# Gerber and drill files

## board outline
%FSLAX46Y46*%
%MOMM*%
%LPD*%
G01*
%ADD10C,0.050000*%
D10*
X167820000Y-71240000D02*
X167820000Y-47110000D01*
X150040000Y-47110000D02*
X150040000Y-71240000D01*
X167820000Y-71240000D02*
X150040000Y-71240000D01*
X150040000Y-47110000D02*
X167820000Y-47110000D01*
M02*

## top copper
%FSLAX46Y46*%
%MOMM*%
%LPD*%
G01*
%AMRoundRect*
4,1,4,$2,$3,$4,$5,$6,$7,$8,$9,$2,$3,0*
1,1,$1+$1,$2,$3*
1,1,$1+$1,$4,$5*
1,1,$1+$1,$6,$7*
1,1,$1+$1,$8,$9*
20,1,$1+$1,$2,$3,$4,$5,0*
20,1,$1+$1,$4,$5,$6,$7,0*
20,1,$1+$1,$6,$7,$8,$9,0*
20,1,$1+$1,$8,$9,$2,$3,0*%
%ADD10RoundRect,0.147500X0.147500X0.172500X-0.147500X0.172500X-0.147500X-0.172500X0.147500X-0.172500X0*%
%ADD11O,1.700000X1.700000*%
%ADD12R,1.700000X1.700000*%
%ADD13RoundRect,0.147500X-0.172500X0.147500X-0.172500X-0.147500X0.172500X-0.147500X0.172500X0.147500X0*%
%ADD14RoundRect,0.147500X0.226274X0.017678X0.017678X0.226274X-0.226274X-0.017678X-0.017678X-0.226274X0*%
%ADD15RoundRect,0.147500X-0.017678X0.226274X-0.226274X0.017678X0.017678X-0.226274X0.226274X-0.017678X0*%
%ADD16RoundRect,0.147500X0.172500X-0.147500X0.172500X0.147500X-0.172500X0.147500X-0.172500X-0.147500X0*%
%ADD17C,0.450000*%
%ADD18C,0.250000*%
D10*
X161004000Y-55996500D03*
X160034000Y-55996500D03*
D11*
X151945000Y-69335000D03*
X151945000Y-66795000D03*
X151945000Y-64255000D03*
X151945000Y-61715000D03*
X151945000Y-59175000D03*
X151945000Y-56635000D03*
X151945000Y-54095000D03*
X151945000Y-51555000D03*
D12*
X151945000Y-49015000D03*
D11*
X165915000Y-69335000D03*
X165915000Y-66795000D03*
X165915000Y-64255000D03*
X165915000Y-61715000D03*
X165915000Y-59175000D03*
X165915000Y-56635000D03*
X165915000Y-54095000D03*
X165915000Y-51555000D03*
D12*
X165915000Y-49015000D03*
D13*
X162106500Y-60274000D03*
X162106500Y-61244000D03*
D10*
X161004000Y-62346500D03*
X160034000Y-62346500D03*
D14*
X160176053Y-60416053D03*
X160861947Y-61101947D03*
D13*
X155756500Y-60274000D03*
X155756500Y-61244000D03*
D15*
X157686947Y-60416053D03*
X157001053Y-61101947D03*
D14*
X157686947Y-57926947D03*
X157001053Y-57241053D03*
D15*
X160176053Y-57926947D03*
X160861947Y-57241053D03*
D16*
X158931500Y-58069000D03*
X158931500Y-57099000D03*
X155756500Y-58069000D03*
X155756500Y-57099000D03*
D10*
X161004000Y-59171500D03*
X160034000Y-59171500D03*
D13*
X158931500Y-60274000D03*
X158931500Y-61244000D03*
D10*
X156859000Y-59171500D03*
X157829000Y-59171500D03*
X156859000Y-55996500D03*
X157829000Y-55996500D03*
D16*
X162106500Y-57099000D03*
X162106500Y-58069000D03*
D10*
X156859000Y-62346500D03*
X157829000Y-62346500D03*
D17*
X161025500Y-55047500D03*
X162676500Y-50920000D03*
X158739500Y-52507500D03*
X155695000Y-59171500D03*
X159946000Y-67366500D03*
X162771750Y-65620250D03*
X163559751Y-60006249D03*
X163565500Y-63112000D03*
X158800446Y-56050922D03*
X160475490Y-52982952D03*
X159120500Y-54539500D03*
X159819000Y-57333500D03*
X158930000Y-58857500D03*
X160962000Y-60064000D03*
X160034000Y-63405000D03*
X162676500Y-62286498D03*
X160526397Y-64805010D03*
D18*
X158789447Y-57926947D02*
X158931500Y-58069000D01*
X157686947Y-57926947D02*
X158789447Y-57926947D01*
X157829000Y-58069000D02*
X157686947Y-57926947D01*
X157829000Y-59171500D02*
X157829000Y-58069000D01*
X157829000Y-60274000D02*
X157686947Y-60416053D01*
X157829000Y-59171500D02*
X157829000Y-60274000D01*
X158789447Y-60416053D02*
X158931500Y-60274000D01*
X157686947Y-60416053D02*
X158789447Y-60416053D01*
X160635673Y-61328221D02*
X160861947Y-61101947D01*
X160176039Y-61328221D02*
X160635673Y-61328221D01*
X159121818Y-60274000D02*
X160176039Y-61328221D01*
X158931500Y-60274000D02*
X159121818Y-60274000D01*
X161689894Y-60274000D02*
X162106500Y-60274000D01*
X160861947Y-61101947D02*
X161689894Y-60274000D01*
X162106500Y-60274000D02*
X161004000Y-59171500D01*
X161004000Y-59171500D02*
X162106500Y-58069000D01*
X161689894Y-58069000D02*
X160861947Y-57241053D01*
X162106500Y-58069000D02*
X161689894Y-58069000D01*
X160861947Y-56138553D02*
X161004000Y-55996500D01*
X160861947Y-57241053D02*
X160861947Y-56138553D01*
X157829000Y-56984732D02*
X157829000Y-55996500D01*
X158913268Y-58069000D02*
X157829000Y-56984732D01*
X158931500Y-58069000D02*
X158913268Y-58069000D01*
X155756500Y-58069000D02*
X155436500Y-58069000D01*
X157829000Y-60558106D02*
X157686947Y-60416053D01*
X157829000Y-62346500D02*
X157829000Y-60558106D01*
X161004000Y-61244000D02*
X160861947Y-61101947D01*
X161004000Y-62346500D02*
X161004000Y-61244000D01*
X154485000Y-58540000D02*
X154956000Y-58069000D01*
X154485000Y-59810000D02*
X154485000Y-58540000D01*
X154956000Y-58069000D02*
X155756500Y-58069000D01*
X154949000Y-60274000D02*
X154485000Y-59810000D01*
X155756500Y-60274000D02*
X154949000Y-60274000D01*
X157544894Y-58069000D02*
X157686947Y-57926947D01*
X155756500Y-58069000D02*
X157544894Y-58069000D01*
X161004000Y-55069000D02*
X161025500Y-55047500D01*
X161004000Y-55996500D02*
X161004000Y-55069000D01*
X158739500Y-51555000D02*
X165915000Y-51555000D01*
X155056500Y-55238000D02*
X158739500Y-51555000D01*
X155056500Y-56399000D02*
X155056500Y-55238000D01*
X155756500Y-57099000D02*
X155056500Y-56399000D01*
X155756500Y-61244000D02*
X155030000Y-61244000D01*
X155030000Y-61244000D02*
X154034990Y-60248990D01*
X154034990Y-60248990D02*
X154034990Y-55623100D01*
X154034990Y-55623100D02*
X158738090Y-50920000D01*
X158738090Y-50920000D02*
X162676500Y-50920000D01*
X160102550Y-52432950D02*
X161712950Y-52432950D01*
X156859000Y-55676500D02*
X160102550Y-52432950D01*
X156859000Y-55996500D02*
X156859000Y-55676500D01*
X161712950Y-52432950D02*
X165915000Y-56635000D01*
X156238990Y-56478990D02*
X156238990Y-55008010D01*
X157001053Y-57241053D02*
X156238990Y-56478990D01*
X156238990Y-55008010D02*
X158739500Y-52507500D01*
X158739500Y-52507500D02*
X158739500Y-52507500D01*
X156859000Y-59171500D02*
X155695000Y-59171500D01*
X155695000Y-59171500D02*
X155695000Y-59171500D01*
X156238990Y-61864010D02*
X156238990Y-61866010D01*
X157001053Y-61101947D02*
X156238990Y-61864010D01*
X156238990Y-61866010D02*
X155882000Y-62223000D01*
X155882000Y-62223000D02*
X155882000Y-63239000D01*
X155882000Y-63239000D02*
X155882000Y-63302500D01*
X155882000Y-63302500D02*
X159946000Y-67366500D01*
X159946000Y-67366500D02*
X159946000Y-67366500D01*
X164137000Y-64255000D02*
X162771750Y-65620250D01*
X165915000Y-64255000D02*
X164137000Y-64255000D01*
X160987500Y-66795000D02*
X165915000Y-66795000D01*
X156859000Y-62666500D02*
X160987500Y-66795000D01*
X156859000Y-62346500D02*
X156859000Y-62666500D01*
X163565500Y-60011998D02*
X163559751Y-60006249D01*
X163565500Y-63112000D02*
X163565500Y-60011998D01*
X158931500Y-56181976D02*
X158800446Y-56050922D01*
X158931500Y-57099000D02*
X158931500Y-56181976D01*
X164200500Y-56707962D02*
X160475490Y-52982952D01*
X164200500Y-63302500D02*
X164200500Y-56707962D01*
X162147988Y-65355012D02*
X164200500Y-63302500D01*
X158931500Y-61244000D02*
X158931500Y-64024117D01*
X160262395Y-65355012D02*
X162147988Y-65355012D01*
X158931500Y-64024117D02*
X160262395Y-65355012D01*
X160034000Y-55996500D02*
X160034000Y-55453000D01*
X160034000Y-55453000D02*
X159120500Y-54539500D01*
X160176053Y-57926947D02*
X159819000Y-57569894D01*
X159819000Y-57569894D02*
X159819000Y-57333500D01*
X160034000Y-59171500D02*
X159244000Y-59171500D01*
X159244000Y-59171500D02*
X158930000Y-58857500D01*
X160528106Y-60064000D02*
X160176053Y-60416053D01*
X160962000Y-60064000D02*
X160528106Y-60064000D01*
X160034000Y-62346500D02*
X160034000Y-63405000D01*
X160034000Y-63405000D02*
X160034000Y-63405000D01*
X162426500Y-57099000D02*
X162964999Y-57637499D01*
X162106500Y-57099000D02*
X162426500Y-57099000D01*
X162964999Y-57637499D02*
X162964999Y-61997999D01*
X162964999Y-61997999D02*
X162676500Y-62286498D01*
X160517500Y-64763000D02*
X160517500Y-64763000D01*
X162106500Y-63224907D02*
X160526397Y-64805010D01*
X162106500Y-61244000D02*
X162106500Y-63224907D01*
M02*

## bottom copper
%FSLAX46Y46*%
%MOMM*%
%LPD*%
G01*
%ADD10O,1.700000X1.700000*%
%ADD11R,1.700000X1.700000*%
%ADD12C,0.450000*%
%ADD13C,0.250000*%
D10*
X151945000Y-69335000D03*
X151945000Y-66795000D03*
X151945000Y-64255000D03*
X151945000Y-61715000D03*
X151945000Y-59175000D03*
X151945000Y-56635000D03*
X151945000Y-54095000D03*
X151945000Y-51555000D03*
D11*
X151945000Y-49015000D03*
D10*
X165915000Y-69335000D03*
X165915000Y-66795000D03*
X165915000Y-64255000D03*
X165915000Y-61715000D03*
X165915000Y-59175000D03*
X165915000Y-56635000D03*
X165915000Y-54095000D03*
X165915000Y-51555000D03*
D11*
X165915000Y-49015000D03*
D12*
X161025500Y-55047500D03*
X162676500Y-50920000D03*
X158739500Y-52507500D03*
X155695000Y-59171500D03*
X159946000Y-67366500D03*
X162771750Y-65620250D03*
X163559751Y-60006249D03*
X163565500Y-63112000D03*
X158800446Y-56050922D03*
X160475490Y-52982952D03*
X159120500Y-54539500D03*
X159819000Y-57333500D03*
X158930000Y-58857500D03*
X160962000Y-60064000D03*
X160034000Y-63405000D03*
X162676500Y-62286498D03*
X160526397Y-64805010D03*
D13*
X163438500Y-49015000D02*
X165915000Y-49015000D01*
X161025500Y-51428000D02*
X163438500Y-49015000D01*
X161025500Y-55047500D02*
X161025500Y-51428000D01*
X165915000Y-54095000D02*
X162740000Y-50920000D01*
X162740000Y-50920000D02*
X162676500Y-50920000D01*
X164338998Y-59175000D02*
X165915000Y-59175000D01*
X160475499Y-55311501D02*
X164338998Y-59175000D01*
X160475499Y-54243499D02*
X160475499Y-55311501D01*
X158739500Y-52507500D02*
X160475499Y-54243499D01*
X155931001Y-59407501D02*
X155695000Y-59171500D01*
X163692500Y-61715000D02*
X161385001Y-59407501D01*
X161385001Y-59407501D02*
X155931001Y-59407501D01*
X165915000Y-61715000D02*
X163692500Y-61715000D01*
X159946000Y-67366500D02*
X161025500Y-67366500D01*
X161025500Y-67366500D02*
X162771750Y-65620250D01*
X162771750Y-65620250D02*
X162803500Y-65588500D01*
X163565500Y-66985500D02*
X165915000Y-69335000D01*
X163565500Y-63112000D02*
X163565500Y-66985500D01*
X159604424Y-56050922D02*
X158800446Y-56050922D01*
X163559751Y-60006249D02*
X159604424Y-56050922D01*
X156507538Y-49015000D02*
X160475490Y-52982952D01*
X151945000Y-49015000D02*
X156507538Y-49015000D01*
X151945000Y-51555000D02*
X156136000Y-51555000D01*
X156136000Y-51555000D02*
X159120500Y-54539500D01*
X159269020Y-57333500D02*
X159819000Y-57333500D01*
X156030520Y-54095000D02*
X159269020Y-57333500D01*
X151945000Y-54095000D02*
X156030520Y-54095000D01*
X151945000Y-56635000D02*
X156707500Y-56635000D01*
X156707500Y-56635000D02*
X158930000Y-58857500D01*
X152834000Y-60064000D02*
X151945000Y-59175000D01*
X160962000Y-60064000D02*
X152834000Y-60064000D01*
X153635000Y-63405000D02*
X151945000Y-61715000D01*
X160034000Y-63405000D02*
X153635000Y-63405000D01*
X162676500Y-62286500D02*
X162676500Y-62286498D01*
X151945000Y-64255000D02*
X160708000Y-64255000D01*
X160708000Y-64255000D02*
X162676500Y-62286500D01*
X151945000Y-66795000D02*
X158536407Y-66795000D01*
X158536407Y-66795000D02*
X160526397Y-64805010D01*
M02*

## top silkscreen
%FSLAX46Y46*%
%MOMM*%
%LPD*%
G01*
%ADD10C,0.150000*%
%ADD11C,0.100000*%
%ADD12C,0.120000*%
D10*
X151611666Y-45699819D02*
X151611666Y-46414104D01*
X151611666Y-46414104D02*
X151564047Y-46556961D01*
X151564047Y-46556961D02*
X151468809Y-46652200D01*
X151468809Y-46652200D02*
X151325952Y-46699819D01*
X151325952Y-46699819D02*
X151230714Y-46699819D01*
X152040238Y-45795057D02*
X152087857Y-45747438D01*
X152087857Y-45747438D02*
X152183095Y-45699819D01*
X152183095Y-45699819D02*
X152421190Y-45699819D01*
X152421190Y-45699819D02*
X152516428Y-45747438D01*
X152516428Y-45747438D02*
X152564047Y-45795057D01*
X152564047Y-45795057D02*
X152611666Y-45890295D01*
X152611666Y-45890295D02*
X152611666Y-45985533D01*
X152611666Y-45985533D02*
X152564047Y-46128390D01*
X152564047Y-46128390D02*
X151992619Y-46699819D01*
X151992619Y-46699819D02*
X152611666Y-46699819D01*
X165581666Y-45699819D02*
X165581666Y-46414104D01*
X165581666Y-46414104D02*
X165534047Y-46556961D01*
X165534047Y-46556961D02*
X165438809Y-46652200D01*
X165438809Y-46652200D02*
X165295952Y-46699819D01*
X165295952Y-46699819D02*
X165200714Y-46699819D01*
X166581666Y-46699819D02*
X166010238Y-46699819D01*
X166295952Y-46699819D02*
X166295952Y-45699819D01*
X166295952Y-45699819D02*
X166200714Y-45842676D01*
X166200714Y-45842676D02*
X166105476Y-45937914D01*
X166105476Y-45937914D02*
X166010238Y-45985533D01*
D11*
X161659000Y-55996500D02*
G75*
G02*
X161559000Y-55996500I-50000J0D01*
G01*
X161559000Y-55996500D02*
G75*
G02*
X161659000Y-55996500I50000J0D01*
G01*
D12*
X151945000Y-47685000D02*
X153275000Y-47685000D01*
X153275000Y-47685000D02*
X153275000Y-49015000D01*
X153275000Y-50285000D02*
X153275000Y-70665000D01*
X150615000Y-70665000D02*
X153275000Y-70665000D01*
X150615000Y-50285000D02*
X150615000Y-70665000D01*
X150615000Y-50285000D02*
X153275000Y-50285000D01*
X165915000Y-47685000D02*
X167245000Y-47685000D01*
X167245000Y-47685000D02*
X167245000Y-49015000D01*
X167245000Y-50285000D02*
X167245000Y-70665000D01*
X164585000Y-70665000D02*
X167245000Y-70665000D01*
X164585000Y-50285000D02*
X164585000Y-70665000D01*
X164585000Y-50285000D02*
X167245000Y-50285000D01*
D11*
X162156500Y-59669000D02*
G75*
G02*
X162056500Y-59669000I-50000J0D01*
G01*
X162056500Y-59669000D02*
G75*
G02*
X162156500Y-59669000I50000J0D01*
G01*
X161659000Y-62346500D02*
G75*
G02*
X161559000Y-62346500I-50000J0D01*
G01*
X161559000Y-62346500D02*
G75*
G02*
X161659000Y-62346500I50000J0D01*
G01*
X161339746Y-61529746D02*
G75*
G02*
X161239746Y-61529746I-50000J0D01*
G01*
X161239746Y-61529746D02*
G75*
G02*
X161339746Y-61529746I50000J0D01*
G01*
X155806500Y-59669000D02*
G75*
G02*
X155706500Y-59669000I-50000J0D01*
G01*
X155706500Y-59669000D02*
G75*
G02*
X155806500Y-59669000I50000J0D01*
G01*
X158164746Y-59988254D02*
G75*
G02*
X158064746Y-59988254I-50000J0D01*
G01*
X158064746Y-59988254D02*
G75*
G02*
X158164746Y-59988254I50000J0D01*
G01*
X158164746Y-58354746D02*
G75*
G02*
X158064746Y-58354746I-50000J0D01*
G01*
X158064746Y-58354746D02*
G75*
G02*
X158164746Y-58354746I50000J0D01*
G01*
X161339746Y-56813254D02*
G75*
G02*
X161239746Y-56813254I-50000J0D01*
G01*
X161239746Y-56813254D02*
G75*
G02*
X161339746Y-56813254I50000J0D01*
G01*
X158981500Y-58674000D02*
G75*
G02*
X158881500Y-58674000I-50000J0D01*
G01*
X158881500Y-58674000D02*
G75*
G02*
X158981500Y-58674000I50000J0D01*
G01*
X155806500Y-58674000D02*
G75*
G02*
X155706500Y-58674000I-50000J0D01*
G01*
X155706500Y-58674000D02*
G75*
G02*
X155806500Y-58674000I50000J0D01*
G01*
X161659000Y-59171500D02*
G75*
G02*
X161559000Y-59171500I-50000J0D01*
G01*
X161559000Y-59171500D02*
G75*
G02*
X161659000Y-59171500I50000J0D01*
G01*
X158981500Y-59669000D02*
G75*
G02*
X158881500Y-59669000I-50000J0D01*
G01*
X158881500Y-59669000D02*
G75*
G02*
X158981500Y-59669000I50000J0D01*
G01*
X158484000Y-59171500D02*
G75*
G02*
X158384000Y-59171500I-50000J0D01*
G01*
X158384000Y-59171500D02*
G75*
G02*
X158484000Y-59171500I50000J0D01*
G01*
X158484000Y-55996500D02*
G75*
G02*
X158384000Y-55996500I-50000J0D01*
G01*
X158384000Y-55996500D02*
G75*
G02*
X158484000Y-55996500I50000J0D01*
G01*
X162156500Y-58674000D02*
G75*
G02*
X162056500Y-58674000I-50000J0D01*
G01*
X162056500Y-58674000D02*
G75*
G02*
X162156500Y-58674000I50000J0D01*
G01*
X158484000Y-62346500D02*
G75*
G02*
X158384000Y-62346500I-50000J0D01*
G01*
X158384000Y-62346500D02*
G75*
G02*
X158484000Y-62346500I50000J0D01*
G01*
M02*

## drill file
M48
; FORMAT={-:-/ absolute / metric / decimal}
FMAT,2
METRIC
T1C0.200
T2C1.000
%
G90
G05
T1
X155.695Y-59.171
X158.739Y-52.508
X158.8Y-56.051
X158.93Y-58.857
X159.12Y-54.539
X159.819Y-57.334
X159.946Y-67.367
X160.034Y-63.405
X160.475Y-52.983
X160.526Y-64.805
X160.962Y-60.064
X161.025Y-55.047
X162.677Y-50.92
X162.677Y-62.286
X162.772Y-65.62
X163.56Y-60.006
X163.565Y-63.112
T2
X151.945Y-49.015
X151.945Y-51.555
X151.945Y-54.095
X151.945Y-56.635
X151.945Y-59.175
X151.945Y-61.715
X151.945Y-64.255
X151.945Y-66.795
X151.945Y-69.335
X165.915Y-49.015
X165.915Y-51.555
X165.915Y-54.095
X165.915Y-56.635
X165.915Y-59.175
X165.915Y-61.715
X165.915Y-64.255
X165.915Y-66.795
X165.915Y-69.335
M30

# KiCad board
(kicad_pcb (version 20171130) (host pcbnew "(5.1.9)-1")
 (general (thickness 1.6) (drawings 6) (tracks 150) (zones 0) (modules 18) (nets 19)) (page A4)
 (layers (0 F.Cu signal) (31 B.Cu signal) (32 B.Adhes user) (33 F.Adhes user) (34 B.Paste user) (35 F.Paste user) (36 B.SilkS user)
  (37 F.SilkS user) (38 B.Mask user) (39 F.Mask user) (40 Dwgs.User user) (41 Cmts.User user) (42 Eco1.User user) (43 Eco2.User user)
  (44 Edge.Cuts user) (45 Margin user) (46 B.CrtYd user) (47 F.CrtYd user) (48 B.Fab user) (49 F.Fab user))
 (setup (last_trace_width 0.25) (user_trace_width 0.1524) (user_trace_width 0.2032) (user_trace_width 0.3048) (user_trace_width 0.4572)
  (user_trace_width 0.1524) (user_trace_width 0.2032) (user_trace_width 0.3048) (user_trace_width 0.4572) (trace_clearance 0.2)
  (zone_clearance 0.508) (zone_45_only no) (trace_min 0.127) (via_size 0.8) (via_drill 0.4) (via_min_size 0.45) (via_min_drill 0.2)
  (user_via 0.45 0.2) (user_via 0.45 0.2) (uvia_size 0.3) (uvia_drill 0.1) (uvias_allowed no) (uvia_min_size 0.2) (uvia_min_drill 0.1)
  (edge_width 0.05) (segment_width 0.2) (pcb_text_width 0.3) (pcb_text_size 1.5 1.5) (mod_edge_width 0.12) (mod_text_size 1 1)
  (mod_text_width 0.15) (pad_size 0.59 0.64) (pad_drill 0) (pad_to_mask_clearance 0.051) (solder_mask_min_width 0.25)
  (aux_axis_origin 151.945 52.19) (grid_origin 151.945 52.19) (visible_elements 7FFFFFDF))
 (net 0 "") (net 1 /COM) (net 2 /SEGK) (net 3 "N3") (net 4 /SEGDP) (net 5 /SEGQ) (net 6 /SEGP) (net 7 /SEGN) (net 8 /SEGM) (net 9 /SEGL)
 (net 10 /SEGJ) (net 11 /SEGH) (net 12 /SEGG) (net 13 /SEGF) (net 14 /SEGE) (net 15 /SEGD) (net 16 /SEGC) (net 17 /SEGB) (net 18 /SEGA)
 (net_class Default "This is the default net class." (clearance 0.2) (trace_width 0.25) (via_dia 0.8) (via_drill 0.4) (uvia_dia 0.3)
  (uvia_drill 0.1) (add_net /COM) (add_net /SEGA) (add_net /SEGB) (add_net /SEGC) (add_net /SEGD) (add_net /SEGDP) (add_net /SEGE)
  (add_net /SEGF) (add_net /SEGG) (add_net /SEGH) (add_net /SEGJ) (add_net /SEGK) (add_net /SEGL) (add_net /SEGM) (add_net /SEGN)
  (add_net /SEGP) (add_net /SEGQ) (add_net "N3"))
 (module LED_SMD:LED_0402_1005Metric (layer F.Cu) (at 160.519 55.9965 180)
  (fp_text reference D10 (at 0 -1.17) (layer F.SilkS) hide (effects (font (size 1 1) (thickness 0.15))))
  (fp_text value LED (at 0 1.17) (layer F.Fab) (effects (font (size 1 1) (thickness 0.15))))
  (fp_circle (center -1.09 0) (end -1.04 0) (layer F.SilkS) (width 0.1))
  (pad 1 smd roundrect (at -0.485 0 180) (size 0.59 0.64) (layers F.Cu F.Paste F.Mask) (roundrect_rratio 0.25) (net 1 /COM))
  (pad 2 smd roundrect (at 0.485 0 180) (size 0.59 0.64) (layers F.Cu F.Paste F.Mask) (roundrect_rratio 0.25) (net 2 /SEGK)))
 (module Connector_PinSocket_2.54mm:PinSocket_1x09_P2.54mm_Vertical (layer F.Cu) (at 151.945 49.015)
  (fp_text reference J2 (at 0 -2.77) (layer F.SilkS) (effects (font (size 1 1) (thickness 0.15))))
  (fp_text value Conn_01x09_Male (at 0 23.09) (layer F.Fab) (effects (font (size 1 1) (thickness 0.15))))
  (fp_line (start 0 -1.33) (end 1.33 -1.33) (layer F.SilkS) (width 0.12))
  (fp_line (start 1.33 -1.33) (end 1.33 0) (layer F.SilkS) (width 0.12))
  (fp_line (start 1.33 1.27) (end 1.33 21.65) (layer F.SilkS) (width 0.12))
  (fp_line (start -1.33 21.65) (end 1.33 21.65) (layer F.SilkS) (width 0.12))
  (fp_line (start -1.33 1.27) (end -1.33 21.65) (layer F.SilkS) (width 0.12))
  (fp_line (start -1.33 1.27) (end 1.33 1.27) (layer F.SilkS) (width 0.12))
  (pad 9 thru_hole oval (at 0 20.32) (size 1.7 1.7) (drill 1) (layers *.Cu *.Mask) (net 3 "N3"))
  (pad 8 thru_hole oval (at 0 17.78) (size 1.7 1.7) (drill 1) (layers *.Cu *.Mask) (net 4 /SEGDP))
  (pad 7 thru_hole oval (at 0 15.24) (size 1.7 1.7) (drill 1) (layers *.Cu *.Mask) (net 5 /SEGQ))
  (pad 6 thru_hole oval (at 0 12.7) (size 1.7 1.7) (drill 1) (layers *.Cu *.Mask) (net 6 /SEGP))
  (pad 5 thru_hole oval (at 0 10.16) (size 1.7 1.7) (drill 1) (layers *.Cu *.Mask) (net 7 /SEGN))
  (pad 4 thru_hole oval (at 0 7.62) (size 1.7 1.7) (drill 1) (layers *.Cu *.Mask) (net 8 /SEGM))
  (pad 3 thru_hole oval (at 0 5.08) (size 1.7 1.7) (drill 1) (layers *.Cu *.Mask) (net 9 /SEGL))
  (pad 2 thru_hole oval (at 0 2.54) (size 1.7 1.7) (drill 1) (layers *.Cu *.Mask) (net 2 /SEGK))
  (pad 1 thru_hole rect (at 0 0) (size 1.7 1.7) (drill 1) (layers *.Cu *.Mask) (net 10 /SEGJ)))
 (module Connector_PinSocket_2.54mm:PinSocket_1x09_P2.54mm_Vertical (layer F.Cu) (at 165.915 49.015)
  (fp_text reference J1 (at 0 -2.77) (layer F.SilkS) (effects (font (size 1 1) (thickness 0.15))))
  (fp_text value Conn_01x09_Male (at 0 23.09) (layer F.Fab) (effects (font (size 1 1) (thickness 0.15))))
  (fp_line (start 0 -1.33) (end 1.33 -1.33) (layer F.SilkS) (width 0.12))
  (fp_line (start 1.33 -1.33) (end 1.33 0) (layer F.SilkS) (width 0.12))
  (fp_line (start 1.33 1.27) (end 1.33 21.65) (layer F.SilkS) (width 0.12))
  (fp_line (start -1.33 21.65) (end 1.33 21.65) (layer F.SilkS) (width 0.12))
  (fp_line (start -1.33 1.27) (end -1.33 21.65) (layer F.SilkS) (width 0.12))
  (fp_line (start -1.33 1.27) (end 1.33 1.27) (layer F.SilkS) (width 0.12))
  (pad 9 thru_hole oval (at 0 20.32) (size 1.7 1.7) (drill 1) (layers *.Cu *.Mask) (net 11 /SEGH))
  (pad 8 thru_hole oval (at 0 17.78) (size 1.7 1.7) (drill 1) (layers *.Cu *.Mask) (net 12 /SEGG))
  (pad 7 thru_hole oval (at 0 15.24) (size 1.7 1.7) (drill 1) (layers *.Cu *.Mask) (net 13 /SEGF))
  (pad 6 thru_hole oval (at 0 12.7) (size 1.7 1.7) (drill 1) (layers *.Cu *.Mask) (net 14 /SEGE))
  (pad 5 thru_hole oval (at 0 10.16) (size 1.7 1.7) (drill 1) (layers *.Cu *.Mask) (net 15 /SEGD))
  (pad 4 thru_hole oval (at 0 7.62) (size 1.7 1.7) (drill 1) (layers *.Cu *.Mask) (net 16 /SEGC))
  (pad 3 thru_hole oval (at 0 5.08) (size 1.7 1.7) (drill 1) (layers *.Cu *.Mask) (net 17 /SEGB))
  (pad 2 thru_hole oval (at 0 2.54) (size 1.7 1.7) (drill 1) (layers *.Cu *.Mask) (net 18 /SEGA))
  (pad 1 thru_hole rect (at 0 0) (size 1.7 1.7) (drill 1) (layers *.Cu *.Mask) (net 1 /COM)))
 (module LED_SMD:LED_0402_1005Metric (layer F.Cu) (at 162.1065 60.759 270)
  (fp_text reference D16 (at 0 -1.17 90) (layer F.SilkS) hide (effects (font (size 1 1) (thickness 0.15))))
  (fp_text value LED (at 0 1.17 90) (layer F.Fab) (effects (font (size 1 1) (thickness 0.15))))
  (fp_circle (center -1.09 0) (end -1.04 0) (layer F.SilkS) (width 0.1))
  (pad 1 smd roundrect (at -0.485 0 270) (size 0.59 0.64) (layers F.Cu F.Paste F.Mask) (roundrect_rratio 0.25) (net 1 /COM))
  (pad 2 smd roundrect (at 0.485 0 270) (size 0.59 0.64) (layers F.Cu F.Paste F.Mask) (roundrect_rratio 0.25) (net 4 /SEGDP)))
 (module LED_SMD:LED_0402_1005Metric (layer F.Cu) (at 160.519 62.3465 180)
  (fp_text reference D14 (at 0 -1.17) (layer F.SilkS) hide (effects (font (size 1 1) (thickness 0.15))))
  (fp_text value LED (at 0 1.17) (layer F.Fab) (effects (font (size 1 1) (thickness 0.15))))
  (fp_circle (center -1.09 0) (end -1.04 0) (layer F.SilkS) (width 0.1))
  (pad 1 smd roundrect (at -0.485 0 180) (size 0.59 0.64) (layers F.Cu F.Paste F.Mask) (roundrect_rratio 0.25) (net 1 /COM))
  (pad 2 smd roundrect (at 0.485 0 180) (size 0.59 0.64) (layers F.Cu F.Paste F.Mask) (roundrect_rratio 0.25) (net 6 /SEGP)))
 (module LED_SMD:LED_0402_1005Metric (layer F.Cu) (at 160.519 60.759 135)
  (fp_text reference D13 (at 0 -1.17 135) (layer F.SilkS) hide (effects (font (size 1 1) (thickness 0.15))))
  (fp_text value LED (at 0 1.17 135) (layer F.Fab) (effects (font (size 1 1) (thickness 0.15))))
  (fp_circle (center -1.09 0) (end -1.04 0) (layer F.SilkS) (width 0.1))
  (pad 2 smd roundrect (at 0.485 0 135) (size 0.59 0.64) (layers F.Cu F.Paste F.Mask) (roundrect_rratio 0.25) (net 7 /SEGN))
  (pad 1 smd roundrect (at -0.485 0 135) (size 0.59 0.64) (layers F.Cu F.Paste F.Mask) (roundrect_rratio 0.25) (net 1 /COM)))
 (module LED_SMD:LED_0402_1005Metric (layer F.Cu) (at 155.7565 60.759 270)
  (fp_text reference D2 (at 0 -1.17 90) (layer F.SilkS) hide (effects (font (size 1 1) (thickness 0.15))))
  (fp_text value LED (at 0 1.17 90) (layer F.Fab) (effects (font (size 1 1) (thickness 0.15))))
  (fp_circle (center -1.09 0) (end -1.04 0) (layer F.SilkS) (width 0.1))
  (pad 1 smd roundrect (at -0.485 0 270) (size 0.59 0.64) (layers F.Cu F.Paste F.Mask) (roundrect_rratio 0.25) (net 1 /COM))
  (pad 2 smd roundrect (at 0.485 0 270) (size 0.59 0.64) (layers F.Cu F.Paste F.Mask) (roundrect_rratio 0.25) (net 17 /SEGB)))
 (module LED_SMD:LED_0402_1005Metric (layer F.Cu) (at 157.344 60.759 225)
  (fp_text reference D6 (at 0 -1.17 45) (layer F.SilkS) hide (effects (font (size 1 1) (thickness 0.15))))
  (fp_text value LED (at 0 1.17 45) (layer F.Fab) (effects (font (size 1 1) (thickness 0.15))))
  (fp_circle (center -1.09 0) (end -1.04 0) (layer F.SilkS) (width 0.1))
  (pad 1 smd roundrect (at -0.485 0 225) (size 0.59 0.64) (layers F.Cu F.Paste F.Mask) (roundrect_rratio 0.25) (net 1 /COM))
  (pad 2 smd roundrect (at 0.485 0 225) (size 0.59 0.64) (layers F.Cu F.Paste F.Mask) (roundrect_rratio 0.25) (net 13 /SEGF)))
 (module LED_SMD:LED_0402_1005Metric (layer F.Cu) (at 157.344 57.584 135)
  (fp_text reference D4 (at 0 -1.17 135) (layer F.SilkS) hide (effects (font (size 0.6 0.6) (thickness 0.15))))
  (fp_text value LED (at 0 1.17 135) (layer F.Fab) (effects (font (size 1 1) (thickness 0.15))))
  (fp_circle (center -1.09 0) (end -1.04 0) (layer F.SilkS) (width 0.1))
  (pad 1 smd roundrect (at -0.485 0 135) (size 0.59 0.64) (layers F.Cu F.Paste F.Mask) (roundrect_rratio 0.25) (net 1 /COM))
  (pad 2 smd roundrect (at 0.485 0 135) (size 0.59 0.64) (layers F.Cu F.Paste F.Mask) (roundrect_rratio 0.25) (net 15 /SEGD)))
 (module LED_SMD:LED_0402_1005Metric (layer F.Cu) (at 160.519 57.584 225)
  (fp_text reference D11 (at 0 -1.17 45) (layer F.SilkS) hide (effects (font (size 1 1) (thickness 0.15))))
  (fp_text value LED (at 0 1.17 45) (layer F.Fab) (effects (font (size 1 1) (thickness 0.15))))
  (fp_circle (center -1.09 0) (end -1.04 0) (layer F.SilkS) (width 0.1))
  (pad 2 smd roundrect (at 0.485 0 225) (size 0.59 0.64) (layers F.Cu F.Paste F.Mask) (roundrect_rratio 0.25) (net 9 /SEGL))
  (pad 1 smd roundrect (at -0.485 0 225) (size 0.59 0.64) (layers F.Cu F.Paste F.Mask) (roundrect_rratio 0.25) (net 1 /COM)))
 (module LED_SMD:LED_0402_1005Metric (layer F.Cu) (at 158.9315 57.584 90)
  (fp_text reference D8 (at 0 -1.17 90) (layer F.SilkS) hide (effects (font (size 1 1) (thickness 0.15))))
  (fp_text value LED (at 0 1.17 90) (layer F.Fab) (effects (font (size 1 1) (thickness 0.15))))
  (fp_circle (center -1.09 0) (end -1.04 0) (layer F.SilkS) (width 0.1))
  (pad 1 smd roundrect (at -0.485 0 90) (size 0.59 0.64) (layers F.Cu F.Paste F.Mask) (roundrect_rratio 0.25) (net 1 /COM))
  (pad 2 smd roundrect (at 0.485 0 90) (size 0.59 0.64) (layers F.Cu F.Paste F.Mask) (roundrect_rratio 0.25) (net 11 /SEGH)))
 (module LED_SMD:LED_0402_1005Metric (layer F.Cu) (at 155.7565 57.584 90)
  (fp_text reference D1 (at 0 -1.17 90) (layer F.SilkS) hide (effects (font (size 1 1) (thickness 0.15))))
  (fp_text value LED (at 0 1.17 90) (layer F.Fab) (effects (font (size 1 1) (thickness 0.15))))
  (fp_circle (center -1.09 0) (end -1.04 0) (layer F.SilkS) (width 0.1))
  (pad 1 smd roundrect (at -0.485 0 90) (size 0.59 0.64) (layers F.Cu F.Paste F.Mask) (roundrect_rratio 0.25) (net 1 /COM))
  (pad 2 smd roundrect (at 0.485 0 90) (size 0.59 0.64) (layers F.Cu F.Paste F.Mask) (roundrect_rratio 0.25) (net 18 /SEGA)))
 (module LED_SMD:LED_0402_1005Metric (layer F.Cu) (at 160.519 59.1715 180)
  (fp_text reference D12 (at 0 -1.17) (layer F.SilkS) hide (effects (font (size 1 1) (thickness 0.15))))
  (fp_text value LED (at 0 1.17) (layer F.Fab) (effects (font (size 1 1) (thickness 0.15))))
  (fp_circle (center -1.09 0) (end -1.04 0) (layer F.SilkS) (width 0.1))
  (pad 1 smd roundrect (at -0.485 0 180) (size 0.59 0.64) (layers F.Cu F.Paste F.Mask) (roundrect_rratio 0.25) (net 1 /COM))
  (pad 2 smd roundrect (at 0.485 0 180) (size 0.59 0.64) (layers F.Cu F.Paste F.Mask) (roundrect_rratio 0.25) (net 8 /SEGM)))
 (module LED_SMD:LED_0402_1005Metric (layer F.Cu) (at 158.9315 60.759 270)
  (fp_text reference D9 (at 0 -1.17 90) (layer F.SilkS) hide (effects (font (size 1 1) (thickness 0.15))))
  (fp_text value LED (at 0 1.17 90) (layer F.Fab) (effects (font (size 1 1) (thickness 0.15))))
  (fp_circle (center -1.09 0) (end -1.04 0) (layer F.SilkS) (width 0.1))
  (pad 1 smd roundrect (at -0.485 0 270) (size 0.59 0.64) (layers F.Cu F.Paste F.Mask) (roundrect_rratio 0.25) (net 1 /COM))
  (pad 2 smd roundrect (at 0.485 0 270) (size 0.59 0.64) (layers F.Cu F.Paste F.Mask) (roundrect_rratio 0.25) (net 10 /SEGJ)))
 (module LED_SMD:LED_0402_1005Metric (layer F.Cu) (at 157.344 59.1715 180)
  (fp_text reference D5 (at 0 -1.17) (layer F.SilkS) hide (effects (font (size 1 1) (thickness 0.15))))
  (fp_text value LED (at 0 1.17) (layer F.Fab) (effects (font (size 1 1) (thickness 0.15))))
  (fp_circle (center -1.09 0) (end -1.04 0) (layer F.SilkS) (width 0.1))
  (pad 2 smd roundrect (at 0.485 0 180) (size 0.59 0.64) (layers F.Cu F.Paste F.Mask) (roundrect_rratio 0.25) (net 14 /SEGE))
  (pad 1 smd roundrect (at -0.485 0 180) (size 0.59 0.64) (layers F.Cu F.Paste F.Mask) (roundrect_rratio 0.25) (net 1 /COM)))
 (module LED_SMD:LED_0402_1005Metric (layer F.Cu) (at 157.344 55.9965 180)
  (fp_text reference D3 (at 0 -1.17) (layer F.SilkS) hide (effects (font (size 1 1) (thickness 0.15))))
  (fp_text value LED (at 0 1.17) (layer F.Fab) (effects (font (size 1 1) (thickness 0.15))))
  (fp_circle (center -1.09 0) (end -1.04 0) (layer F.SilkS) (width 0.1))
  (pad 2 smd roundrect (at 0.485 0 180) (size 0.59 0.64) (layers F.Cu F.Paste F.Mask) (roundrect_rratio 0.25) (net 16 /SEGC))
  (pad 1 smd roundrect (at -0.485 0 180) (size 0.59 0.64) (layers F.Cu F.Paste F.Mask) (roundrect_rratio 0.25) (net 1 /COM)))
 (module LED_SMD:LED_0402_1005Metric (layer F.Cu) (at 162.1065 57.584 90)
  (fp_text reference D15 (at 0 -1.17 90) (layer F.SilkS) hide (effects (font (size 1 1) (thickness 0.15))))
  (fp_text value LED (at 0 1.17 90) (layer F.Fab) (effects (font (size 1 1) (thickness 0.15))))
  (fp_circle (center -1.09 0) (end -1.04 0) (layer F.SilkS) (width 0.1))
  (pad 2 smd roundrect (at 0.485 0 90) (size 0.59 0.64) (layers F.Cu F.Paste F.Mask) (roundrect_rratio 0.25) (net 5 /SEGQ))
  (pad 1 smd roundrect (at -0.485 0 90) (size 0.59 0.64) (layers F.Cu F.Paste F.Mask) (roundrect_rratio 0.25) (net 1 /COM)))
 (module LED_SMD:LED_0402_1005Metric (layer F.Cu) (at 157.344 62.3465 180)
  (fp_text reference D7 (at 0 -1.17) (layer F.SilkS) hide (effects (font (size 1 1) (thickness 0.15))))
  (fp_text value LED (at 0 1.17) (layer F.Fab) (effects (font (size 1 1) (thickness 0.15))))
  (fp_circle (center -1.09 0) (end -1.04 0) (layer F.SilkS) (width 0.1))
  (pad 2 smd roundrect (at 0.485 0 180) (size 0.59 0.64) (layers F.Cu F.Paste F.Mask) (roundrect_rratio 0.25) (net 12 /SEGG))
  (pad 1 smd roundrect (at -0.485 0 180) (size 0.59 0.64) (layers F.Cu F.Paste F.Mask) (roundrect_rratio 0.25) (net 1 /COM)))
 (gr_line (start 167.82 71.24) (end 167.82 47.11) (layer Edge.Cuts) (width 0.05))
 (gr_line (start 150.04 47.11) (end 150.04 71.24) (layer Edge.Cuts) (width 0.05))
 (gr_line (start 167.82 71.24) (end 150.04 71.24) (layer Edge.Cuts) (width 0.05))
 (gr_line (start 150.04 47.11) (end 167.82 47.11) (layer Edge.Cuts) (width 0.05))
 (via (at 161.0255 55.0475) (size 0.45) (drill 0.2) (layers F.Cu B.Cu) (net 1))
 (segment (start 158.789447 57.926947) (end 158.9315 58.069) (width 0.25) (layer F.Cu) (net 1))
 (segment (start 157.686947 57.926947) (end 158.789447 57.926947) (width 0.25) (layer F.Cu) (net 1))
 (segment (start 157.829 58.069) (end 157.686947 57.926947) (width 0.25) (layer F.Cu) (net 1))
 (segment (start 157.829 59.1715) (end 157.829 58.069) (width 0.25) (layer F.Cu) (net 1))
 (segment (start 157.829 60.274) (end 157.686947 60.416053) (width 0.25) (layer F.Cu) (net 1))
 (segment (start 157.829 59.1715) (end 157.829 60.274) (width 0.25) (layer F.Cu) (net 1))
 (segment (start 158.789447 60.416053) (end 158.9315 60.274) (width 0.25) (layer F.Cu) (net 1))
 (segment (start 157.686947 60.416053) (end 158.789447 60.416053) (width 0.25) (layer F.Cu) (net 1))
 (segment (start 160.635673 61.328221) (end 160.861947 61.101947) (width 0.25) (layer F.Cu) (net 1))
 (segment (start 160.176039 61.328221) (end 160.635673 61.328221) (width 0.25) (layer F.Cu) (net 1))
 (segment (start 159.121818 60.274) (end 160.176039 61.328221) (width 0.25) (layer F.Cu) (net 1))
 (segment (start 158.9315 60.274) (end 159.121818 60.274) (width 0.25) (layer F.Cu) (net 1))
 (segment (start 161.689894 60.274) (end 162.1065 60.274) (width 0.25) (layer F.Cu) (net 1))
 (segment (start 160.861947 61.101947) (end 161.689894 60.274) (width 0.25) (layer F.Cu) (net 1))
 (segment (start 162.1065 60.274) (end 161.004 59.1715) (width 0.25) (layer F.Cu) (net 1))
 (segment (start 161.004 59.1715) (end 162.1065 58.069) (width 0.25) (layer F.Cu) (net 1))
 (segment (start 161.689894 58.069) (end 160.861947 57.241053) (width 0.25) (layer F.Cu) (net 1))
 (segment (start 162.1065 58.069) (end 161.689894 58.069) (width 0.25) (layer F.Cu) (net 1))
 (segment (start 160.861947 56.138553) (end 161.004 55.9965) (width 0.25) (layer F.Cu) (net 1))
 (segment (start 160.861947 57.241053) (end 160.861947 56.138553) (width 0.25) (layer F.Cu) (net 1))
 (segment (start 157.829 56.984732) (end 157.829 55.9965) (width 0.25) (layer F.Cu) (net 1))
 (segment (start 158.913268 58.069) (end 157.829 56.984732) (width 0.25) (layer F.Cu) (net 1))
 (segment (start 158.9315 58.069) (end 158.913268 58.069) (width 0.25) (layer F.Cu) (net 1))
 (segment (start 155.7565 58.069) (end 155.4365 58.069) (width 0.25) (layer F.Cu) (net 1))
 (segment (start 157.829 60.558106) (end 157.686947 60.416053) (width 0.25) (layer F.Cu) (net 1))
 (segment (start 157.829 62.3465) (end 157.829 60.558106) (width 0.25) (layer F.Cu) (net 1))
 (segment (start 161.004 61.244) (end 160.861947 61.101947) (width 0.25) (layer F.Cu) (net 1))
 (segment (start 161.004 62.3465) (end 161.004 61.244) (width 0.25) (layer F.Cu) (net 1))
 (segment (start 154.485 58.54) (end 154.956 58.069) (width 0.25) (layer F.Cu) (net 1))
 (segment (start 154.485 59.81) (end 154.485 58.54) (width 0.25) (layer F.Cu) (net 1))
 (segment (start 154.956 58.069) (end 155.7565 58.069) (width 0.25) (layer F.Cu) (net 1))
 (segment (start 154.949 60.274) (end 154.485 59.81) (width 0.25) (layer F.Cu) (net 1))
 (segment (start 155.7565 60.274) (end 154.949 60.274) (width 0.25) (layer F.Cu) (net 1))
 (segment (start 157.544894 58.069) (end 157.686947 57.926947) (width 0.25) (layer F.Cu) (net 1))
 (segment (start 155.7565 58.069) (end 157.544894 58.069) (width 0.25) (layer F.Cu) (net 1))
 (segment (start 161.004 55.069) (end 161.0255 55.0475) (width 0.25) (layer F.Cu) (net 1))
 (segment (start 161.004 55.9965) (end 161.004 55.069) (width 0.25) (layer F.Cu) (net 1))
 (segment (start 163.4385 49.015) (end 165.915 49.015) (width 0.25) (layer B.Cu) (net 1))
 (segment (start 161.0255 51.428) (end 163.4385 49.015) (width 0.25) (layer B.Cu) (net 1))
 (segment (start 161.0255 55.0475) (end 161.0255 51.428) (width 0.25) (layer B.Cu) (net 1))
 (segment (start 158.7395 51.555) (end 165.915 51.555) (width 0.25) (layer F.Cu) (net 18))
 (segment (start 155.0565 55.238) (end 158.7395 51.555) (width 0.25) (layer F.Cu) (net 18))
 (segment (start 155.0565 56.399) (end 155.0565 55.238) (width 0.25) (layer F.Cu) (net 18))
 (segment (start 155.7565 57.099) (end 155.0565 56.399) (width 0.25) (layer F.Cu) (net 18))
 (via (at 162.6765 50.92) (size 0.45) (drill 0.2) (layers F.Cu B.Cu) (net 17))
 (segment (start 165.915 54.095) (end 162.74 50.92) (width 0.25) (layer B.Cu) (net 17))
 (segment (start 162.74 50.92) (end 162.6765 50.92) (width 0.25) (layer B.Cu) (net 17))
 (segment (start 155.7565 61.244) (end 155.03 61.244) (width 0.25) (layer F.Cu) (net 17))
 (segment (start 155.03 61.244) (end 154.03499 60.24899) (width 0.25) (layer F.Cu) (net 17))
 (segment (start 154.03499 60.24899) (end 154.03499 55.6231) (width 0.25) (layer F.Cu) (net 17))
 (segment (start 154.03499 55.6231) (end 158.73809 50.92) (width 0.25) (layer F.Cu) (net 17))
 (segment (start 158.73809 50.92) (end 162.6765 50.92) (width 0.25) (layer F.Cu) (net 17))
 (segment (start 160.10255 52.43295) (end 161.71295 52.43295) (width 0.25) (layer F.Cu) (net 16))
 (segment (start 156.859 55.6765) (end 160.10255 52.43295) (width 0.25) (layer F.Cu) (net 16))
 (segment (start 156.859 55.9965) (end 156.859 55.6765) (width 0.25) (layer F.Cu) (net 16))
 (segment (start 161.71295 52.43295) (end 165.915 56.635) (width 0.25) (layer F.Cu) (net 16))
 (segment (start 156.23899 56.47899) (end 156.23899 55.00801) (width 0.25) (layer F.Cu) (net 15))
 (segment (start 157.001053 57.241053) (end 156.23899 56.47899) (width 0.25) (layer F.Cu) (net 15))
 (segment (start 156.23899 55.00801) (end 158.7395 52.5075) (width 0.25) (layer F.Cu) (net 15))
 (segment (start 158.7395 52.5075) (end 158.7395 52.5075) (width 0.25) (layer F.Cu) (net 15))
 (via (at 158.7395 52.5075) (size 0.45) (drill 0.2) (layers F.Cu B.Cu) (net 15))
 (segment (start 164.338998 59.175) (end 165.915 59.175) (width 0.25) (layer B.Cu) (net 15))
 (segment (start 160.475499 55.311501) (end 164.338998 59.175) (width 0.25) (layer B.Cu) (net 15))
 (segment (start 160.475499 54.243499) (end 160.475499 55.311501) (width 0.25) (layer B.Cu) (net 15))
 (segment (start 158.7395 52.5075) (end 160.475499 54.243499) (width 0.25) (layer B.Cu) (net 15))
 (segment (start 156.859 59.1715) (end 155.695 59.1715) (width 0.25) (layer F.Cu) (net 14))
 (segment (start 155.695 59.1715) (end 155.695 59.1715) (width 0.25) (layer F.Cu) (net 14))
 (via (at 155.695 59.1715) (size 0.45) (drill 0.2) (layers F.Cu B.Cu) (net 14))
 (segment (start 155.931001 59.407501) (end 155.695 59.1715) (width 0.25) (layer B.Cu) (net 14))
 (segment (start 163.6925 61.715) (end 161.385001 59.407501) (width 0.25) (layer B.Cu) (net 14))
 (segment (start 161.385001 59.407501) (end 155.931001 59.407501) (width 0.25) (layer B.Cu) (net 14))
 (segment (start 165.915 61.715) (end 163.6925 61.715) (width 0.25) (layer B.Cu) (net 14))
 (segment (start 156.23899 61.86401) (end 156.23899 61.86601) (width 0.25) (layer F.Cu) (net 13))
 (segment (start 157.001053 61.101947) (end 156.23899 61.86401) (width 0.25) (layer F.Cu) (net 13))
 (segment (start 156.23899 61.86601) (end 155.882 62.223) (width 0.25) (layer F.Cu) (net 13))
 (segment (start 155.882 62.223) (end 155.882 63.239) (width 0.25) (layer F.Cu) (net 13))
 (segment (start 155.882 63.239) (end 155.882 63.3025) (width 0.25) (layer F.Cu) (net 13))
 (segment (start 155.882 63.3025) (end 159.946 67.3665) (width 0.25) (layer F.Cu) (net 13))
 (segment (start 159.946 67.3665) (end 159.946 67.3665) (width 0.25) (layer F.Cu) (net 13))
 (via (at 159.946 67.3665) (size 0.45) (drill 0.2) (layers F.Cu B.Cu) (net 13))
 (segment (start 159.946 67.3665) (end 161.0255 67.3665) (width 0.25) (layer B.Cu) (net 13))
 (segment (start 161.0255 67.3665) (end 162.77175 65.62025) (width 0.25) (layer B.Cu) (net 13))
 (segment (start 162.77175 65.62025) (end 162.8035 65.5885) (width 0.25) (layer B.Cu) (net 13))
 (via (at 162.77175 65.62025) (size 0.45) (drill 0.2) (layers F.Cu B.Cu) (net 13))
 (segment (start 164.137 64.255) (end 162.77175 65.62025) (width 0.25) (layer F.Cu) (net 13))
 (segment (start 165.915 64.255) (end 164.137 64.255) (width 0.25) (layer F.Cu) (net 13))
 (segment (start 160.9875 66.795) (end 165.915 66.795) (width 0.25) (layer F.Cu) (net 12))
 (segment (start 156.859 62.6665) (end 160.9875 66.795) (width 0.25) (layer F.Cu) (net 12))
 (segment (start 156.859 62.3465) (end 156.859 62.6665) (width 0.25) (layer F.Cu) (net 12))
 (segment (start 163.5655 66.9855) (end 165.915 69.335) (width 0.25) (layer B.Cu) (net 11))
 (via (at 163.559751 60.006249) (size 0.45) (drill 0.2) (layers F.Cu B.Cu) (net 11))
 (segment (start 163.5655 63.112) (end 163.5655 66.9855) (width 0.25) (layer B.Cu) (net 11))
 (via (at 163.5655 63.112) (size 0.45) (drill 0.2) (layers F.Cu B.Cu) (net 11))
 (segment (start 163.5655 60.011998) (end 163.559751 60.006249) (width 0.25) (layer F.Cu) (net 11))
 (segment (start 163.5655 63.112) (end 163.5655 60.011998) (width 0.25) (layer F.Cu) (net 11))
 (segment (start 158.9315 56.181976) (end 158.800446 56.050922) (width 0.25) (layer F.Cu) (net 11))
 (segment (start 158.9315 57.099) (end 158.9315 56.181976) (width 0.25) (layer F.Cu) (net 11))
 (via (at 158.800446 56.050922) (size 0.45) (drill 0.2) (layers F.Cu B.Cu) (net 11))
 (segment (start 159.604424 56.050922) (end 158.800446 56.050922) (width 0.25) (layer B.Cu) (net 11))
 (segment (start 163.559751 60.006249) (end 159.604424 56.050922) (width 0.25) (layer B.Cu) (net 11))
 (segment (start 164.2005 56.707962) (end 160.47549 52.982952) (width 0.25) (layer F.Cu) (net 10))
 (segment (start 164.2005 63.3025) (end 164.2005 56.707962) (width 0.25) (layer F.Cu) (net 10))
 (segment (start 162.147988 65.355012) (end 164.2005 63.3025) (width 0.25) (layer F.Cu) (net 10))
 (segment (start 158.9315 61.244) (end 158.9315 64.024117) (width 0.25) (layer F.Cu) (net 10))
 (segment (start 156.507538 49.015) (end 160.47549 52.982952) (width 0.25) (layer B.Cu) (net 10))
 (segment (start 151.945 49.015) (end 156.507538 49.015) (width 0.25) (layer B.Cu) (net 10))
 (via (at 160.47549 52.982952) (size 0.45) (drill 0.2) (layers F.Cu B.Cu) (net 10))
 (segment (start 160.262395 65.355012) (end 162.147988 65.355012) (width 0.25) (layer F.Cu) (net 10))
 (segment (start 158.9315 64.024117) (end 160.262395 65.355012) (width 0.25) (layer F.Cu) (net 10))
 (via (at 159.1205 54.5395) (size 0.45) (drill 0.2) (layers F.Cu B.Cu) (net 2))
 (segment (start 160.034 55.9965) (end 160.034 55.453) (width 0.25) (layer F.Cu) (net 2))
 (segment (start 160.034 55.453) (end 159.1205 54.5395) (width 0.25) (layer F.Cu) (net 2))
 (segment (start 151.945 51.555) (end 156.136 51.555) (width 0.25) (layer B.Cu) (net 2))
 (segment (start 156.136 51.555) (end 159.1205 54.5395) (width 0.25) (layer B.Cu) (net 2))
 (via (at 159.819 57.3335) (size 0.45) (drill 0.2) (layers F.Cu B.Cu) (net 9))
 (segment (start 159.26902 57.3335) (end 159.819 57.3335) (width 0.25) (layer B.Cu) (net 9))
 (segment (start 156.03052 54.095) (end 159.26902 57.3335) (width 0.25) (layer B.Cu) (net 9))
 (segment (start 151.945 54.095) (end 156.03052 54.095) (width 0.25) (layer B.Cu) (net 9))
 (segment (start 160.176053 57.926947) (end 159.819 57.569894) (width 0.25) (layer F.Cu) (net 9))
 (segment (start 159.819 57.569894) (end 159.819 57.3335) (width 0.25) (layer F.Cu) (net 9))
 (via (at 158.93 58.8575) (size 0.45) (drill 0.2) (layers F.Cu B.Cu) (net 8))
 (segment (start 151.945 56.635) (end 156.7075 56.635) (width 0.25) (layer B.Cu) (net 8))
 (segment (start 156.7075 56.635) (end 158.93 58.8575) (width 0.25) (layer B.Cu) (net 8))
 (segment (start 160.034 59.1715) (end 159.244 59.1715) (width 0.25) (layer F.Cu) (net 8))
 (segment (start 159.244 59.1715) (end 158.93 58.8575) (width 0.25) (layer F.Cu) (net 8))
 (via (at 160.962 60.064) (size 0.45) (drill 0.2) (layers F.Cu B.Cu) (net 7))
 (segment (start 160.528106 60.064) (end 160.176053 60.416053) (width 0.25) (layer F.Cu) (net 7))
 (segment (start 160.962 60.064) (end 160.528106 60.064) (width 0.25) (layer F.Cu) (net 7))
 (segment (start 152.834 60.064) (end 151.945 59.175) (width 0.25) (layer B.Cu) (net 7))
 (segment (start 160.962 60.064) (end 152.834 60.064) (width 0.25) (layer B.Cu) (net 7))
 (segment (start 160.034 62.3465) (end 160.034 63.405) (width 0.25) (layer F.Cu) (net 6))
 (segment (start 160.034 63.405) (end 160.034 63.405) (width 0.25) (layer F.Cu) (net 6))
 (via (at 160.034 63.405) (size 0.45) (drill 0.2) (layers F.Cu B.Cu) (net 6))
 (segment (start 153.635 63.405) (end 151.945 61.715) (width 0.25) (layer B.Cu) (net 6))
 (segment (start 160.034 63.405) (end 153.635 63.405) (width 0.25) (layer B.Cu) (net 6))
 (via (at 162.6765 62.286498) (size 0.45) (drill 0.2) (layers F.Cu B.Cu) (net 5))
 (segment (start 162.4265 57.099) (end 162.964999 57.637499) (width 0.25) (layer F.Cu) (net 5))
 (segment (start 162.1065 57.099) (end 162.4265 57.099) (width 0.25) (layer F.Cu) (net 5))
 (segment (start 162.964999 57.637499) (end 162.964999 61.997999) (width 0.25) (layer F.Cu) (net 5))
 (segment (start 162.964999 61.997999) (end 162.6765 62.286498) (width 0.25) (layer F.Cu) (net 5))
 (segment (start 162.6765 62.2865) (end 162.6765 62.286498) (width 0.25) (layer B.Cu) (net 5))
 (segment (start 151.945 64.255) (end 160.708 64.255) (width 0.25) (layer B.Cu) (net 5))
 (segment (start 160.708 64.255) (end 162.6765 62.2865) (width 0.25) (layer B.Cu) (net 5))
 (segment (start 160.5175 64.763) (end 160.5175 64.763) (width 0.25) (layer F.Cu) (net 4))
 (via (at 160.526397 64.80501) (size 0.45) (drill 0.2) (layers F.Cu B.Cu) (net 4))
 (segment (start 162.1065 63.224907) (end 160.526397 64.80501) (width 0.25) (layer F.Cu) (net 4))
 (segment (start 151.945 66.795) (end 158.536407 66.795) (width 0.25) (layer B.Cu) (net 4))
 (segment (start 162.1065 61.244) (end 162.1065 63.224907) (width 0.25) (layer F.Cu) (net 4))
 (segment (start 158.536407 66.795) (end 160.526397 64.80501) (width 0.25) (layer B.Cu) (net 4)))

